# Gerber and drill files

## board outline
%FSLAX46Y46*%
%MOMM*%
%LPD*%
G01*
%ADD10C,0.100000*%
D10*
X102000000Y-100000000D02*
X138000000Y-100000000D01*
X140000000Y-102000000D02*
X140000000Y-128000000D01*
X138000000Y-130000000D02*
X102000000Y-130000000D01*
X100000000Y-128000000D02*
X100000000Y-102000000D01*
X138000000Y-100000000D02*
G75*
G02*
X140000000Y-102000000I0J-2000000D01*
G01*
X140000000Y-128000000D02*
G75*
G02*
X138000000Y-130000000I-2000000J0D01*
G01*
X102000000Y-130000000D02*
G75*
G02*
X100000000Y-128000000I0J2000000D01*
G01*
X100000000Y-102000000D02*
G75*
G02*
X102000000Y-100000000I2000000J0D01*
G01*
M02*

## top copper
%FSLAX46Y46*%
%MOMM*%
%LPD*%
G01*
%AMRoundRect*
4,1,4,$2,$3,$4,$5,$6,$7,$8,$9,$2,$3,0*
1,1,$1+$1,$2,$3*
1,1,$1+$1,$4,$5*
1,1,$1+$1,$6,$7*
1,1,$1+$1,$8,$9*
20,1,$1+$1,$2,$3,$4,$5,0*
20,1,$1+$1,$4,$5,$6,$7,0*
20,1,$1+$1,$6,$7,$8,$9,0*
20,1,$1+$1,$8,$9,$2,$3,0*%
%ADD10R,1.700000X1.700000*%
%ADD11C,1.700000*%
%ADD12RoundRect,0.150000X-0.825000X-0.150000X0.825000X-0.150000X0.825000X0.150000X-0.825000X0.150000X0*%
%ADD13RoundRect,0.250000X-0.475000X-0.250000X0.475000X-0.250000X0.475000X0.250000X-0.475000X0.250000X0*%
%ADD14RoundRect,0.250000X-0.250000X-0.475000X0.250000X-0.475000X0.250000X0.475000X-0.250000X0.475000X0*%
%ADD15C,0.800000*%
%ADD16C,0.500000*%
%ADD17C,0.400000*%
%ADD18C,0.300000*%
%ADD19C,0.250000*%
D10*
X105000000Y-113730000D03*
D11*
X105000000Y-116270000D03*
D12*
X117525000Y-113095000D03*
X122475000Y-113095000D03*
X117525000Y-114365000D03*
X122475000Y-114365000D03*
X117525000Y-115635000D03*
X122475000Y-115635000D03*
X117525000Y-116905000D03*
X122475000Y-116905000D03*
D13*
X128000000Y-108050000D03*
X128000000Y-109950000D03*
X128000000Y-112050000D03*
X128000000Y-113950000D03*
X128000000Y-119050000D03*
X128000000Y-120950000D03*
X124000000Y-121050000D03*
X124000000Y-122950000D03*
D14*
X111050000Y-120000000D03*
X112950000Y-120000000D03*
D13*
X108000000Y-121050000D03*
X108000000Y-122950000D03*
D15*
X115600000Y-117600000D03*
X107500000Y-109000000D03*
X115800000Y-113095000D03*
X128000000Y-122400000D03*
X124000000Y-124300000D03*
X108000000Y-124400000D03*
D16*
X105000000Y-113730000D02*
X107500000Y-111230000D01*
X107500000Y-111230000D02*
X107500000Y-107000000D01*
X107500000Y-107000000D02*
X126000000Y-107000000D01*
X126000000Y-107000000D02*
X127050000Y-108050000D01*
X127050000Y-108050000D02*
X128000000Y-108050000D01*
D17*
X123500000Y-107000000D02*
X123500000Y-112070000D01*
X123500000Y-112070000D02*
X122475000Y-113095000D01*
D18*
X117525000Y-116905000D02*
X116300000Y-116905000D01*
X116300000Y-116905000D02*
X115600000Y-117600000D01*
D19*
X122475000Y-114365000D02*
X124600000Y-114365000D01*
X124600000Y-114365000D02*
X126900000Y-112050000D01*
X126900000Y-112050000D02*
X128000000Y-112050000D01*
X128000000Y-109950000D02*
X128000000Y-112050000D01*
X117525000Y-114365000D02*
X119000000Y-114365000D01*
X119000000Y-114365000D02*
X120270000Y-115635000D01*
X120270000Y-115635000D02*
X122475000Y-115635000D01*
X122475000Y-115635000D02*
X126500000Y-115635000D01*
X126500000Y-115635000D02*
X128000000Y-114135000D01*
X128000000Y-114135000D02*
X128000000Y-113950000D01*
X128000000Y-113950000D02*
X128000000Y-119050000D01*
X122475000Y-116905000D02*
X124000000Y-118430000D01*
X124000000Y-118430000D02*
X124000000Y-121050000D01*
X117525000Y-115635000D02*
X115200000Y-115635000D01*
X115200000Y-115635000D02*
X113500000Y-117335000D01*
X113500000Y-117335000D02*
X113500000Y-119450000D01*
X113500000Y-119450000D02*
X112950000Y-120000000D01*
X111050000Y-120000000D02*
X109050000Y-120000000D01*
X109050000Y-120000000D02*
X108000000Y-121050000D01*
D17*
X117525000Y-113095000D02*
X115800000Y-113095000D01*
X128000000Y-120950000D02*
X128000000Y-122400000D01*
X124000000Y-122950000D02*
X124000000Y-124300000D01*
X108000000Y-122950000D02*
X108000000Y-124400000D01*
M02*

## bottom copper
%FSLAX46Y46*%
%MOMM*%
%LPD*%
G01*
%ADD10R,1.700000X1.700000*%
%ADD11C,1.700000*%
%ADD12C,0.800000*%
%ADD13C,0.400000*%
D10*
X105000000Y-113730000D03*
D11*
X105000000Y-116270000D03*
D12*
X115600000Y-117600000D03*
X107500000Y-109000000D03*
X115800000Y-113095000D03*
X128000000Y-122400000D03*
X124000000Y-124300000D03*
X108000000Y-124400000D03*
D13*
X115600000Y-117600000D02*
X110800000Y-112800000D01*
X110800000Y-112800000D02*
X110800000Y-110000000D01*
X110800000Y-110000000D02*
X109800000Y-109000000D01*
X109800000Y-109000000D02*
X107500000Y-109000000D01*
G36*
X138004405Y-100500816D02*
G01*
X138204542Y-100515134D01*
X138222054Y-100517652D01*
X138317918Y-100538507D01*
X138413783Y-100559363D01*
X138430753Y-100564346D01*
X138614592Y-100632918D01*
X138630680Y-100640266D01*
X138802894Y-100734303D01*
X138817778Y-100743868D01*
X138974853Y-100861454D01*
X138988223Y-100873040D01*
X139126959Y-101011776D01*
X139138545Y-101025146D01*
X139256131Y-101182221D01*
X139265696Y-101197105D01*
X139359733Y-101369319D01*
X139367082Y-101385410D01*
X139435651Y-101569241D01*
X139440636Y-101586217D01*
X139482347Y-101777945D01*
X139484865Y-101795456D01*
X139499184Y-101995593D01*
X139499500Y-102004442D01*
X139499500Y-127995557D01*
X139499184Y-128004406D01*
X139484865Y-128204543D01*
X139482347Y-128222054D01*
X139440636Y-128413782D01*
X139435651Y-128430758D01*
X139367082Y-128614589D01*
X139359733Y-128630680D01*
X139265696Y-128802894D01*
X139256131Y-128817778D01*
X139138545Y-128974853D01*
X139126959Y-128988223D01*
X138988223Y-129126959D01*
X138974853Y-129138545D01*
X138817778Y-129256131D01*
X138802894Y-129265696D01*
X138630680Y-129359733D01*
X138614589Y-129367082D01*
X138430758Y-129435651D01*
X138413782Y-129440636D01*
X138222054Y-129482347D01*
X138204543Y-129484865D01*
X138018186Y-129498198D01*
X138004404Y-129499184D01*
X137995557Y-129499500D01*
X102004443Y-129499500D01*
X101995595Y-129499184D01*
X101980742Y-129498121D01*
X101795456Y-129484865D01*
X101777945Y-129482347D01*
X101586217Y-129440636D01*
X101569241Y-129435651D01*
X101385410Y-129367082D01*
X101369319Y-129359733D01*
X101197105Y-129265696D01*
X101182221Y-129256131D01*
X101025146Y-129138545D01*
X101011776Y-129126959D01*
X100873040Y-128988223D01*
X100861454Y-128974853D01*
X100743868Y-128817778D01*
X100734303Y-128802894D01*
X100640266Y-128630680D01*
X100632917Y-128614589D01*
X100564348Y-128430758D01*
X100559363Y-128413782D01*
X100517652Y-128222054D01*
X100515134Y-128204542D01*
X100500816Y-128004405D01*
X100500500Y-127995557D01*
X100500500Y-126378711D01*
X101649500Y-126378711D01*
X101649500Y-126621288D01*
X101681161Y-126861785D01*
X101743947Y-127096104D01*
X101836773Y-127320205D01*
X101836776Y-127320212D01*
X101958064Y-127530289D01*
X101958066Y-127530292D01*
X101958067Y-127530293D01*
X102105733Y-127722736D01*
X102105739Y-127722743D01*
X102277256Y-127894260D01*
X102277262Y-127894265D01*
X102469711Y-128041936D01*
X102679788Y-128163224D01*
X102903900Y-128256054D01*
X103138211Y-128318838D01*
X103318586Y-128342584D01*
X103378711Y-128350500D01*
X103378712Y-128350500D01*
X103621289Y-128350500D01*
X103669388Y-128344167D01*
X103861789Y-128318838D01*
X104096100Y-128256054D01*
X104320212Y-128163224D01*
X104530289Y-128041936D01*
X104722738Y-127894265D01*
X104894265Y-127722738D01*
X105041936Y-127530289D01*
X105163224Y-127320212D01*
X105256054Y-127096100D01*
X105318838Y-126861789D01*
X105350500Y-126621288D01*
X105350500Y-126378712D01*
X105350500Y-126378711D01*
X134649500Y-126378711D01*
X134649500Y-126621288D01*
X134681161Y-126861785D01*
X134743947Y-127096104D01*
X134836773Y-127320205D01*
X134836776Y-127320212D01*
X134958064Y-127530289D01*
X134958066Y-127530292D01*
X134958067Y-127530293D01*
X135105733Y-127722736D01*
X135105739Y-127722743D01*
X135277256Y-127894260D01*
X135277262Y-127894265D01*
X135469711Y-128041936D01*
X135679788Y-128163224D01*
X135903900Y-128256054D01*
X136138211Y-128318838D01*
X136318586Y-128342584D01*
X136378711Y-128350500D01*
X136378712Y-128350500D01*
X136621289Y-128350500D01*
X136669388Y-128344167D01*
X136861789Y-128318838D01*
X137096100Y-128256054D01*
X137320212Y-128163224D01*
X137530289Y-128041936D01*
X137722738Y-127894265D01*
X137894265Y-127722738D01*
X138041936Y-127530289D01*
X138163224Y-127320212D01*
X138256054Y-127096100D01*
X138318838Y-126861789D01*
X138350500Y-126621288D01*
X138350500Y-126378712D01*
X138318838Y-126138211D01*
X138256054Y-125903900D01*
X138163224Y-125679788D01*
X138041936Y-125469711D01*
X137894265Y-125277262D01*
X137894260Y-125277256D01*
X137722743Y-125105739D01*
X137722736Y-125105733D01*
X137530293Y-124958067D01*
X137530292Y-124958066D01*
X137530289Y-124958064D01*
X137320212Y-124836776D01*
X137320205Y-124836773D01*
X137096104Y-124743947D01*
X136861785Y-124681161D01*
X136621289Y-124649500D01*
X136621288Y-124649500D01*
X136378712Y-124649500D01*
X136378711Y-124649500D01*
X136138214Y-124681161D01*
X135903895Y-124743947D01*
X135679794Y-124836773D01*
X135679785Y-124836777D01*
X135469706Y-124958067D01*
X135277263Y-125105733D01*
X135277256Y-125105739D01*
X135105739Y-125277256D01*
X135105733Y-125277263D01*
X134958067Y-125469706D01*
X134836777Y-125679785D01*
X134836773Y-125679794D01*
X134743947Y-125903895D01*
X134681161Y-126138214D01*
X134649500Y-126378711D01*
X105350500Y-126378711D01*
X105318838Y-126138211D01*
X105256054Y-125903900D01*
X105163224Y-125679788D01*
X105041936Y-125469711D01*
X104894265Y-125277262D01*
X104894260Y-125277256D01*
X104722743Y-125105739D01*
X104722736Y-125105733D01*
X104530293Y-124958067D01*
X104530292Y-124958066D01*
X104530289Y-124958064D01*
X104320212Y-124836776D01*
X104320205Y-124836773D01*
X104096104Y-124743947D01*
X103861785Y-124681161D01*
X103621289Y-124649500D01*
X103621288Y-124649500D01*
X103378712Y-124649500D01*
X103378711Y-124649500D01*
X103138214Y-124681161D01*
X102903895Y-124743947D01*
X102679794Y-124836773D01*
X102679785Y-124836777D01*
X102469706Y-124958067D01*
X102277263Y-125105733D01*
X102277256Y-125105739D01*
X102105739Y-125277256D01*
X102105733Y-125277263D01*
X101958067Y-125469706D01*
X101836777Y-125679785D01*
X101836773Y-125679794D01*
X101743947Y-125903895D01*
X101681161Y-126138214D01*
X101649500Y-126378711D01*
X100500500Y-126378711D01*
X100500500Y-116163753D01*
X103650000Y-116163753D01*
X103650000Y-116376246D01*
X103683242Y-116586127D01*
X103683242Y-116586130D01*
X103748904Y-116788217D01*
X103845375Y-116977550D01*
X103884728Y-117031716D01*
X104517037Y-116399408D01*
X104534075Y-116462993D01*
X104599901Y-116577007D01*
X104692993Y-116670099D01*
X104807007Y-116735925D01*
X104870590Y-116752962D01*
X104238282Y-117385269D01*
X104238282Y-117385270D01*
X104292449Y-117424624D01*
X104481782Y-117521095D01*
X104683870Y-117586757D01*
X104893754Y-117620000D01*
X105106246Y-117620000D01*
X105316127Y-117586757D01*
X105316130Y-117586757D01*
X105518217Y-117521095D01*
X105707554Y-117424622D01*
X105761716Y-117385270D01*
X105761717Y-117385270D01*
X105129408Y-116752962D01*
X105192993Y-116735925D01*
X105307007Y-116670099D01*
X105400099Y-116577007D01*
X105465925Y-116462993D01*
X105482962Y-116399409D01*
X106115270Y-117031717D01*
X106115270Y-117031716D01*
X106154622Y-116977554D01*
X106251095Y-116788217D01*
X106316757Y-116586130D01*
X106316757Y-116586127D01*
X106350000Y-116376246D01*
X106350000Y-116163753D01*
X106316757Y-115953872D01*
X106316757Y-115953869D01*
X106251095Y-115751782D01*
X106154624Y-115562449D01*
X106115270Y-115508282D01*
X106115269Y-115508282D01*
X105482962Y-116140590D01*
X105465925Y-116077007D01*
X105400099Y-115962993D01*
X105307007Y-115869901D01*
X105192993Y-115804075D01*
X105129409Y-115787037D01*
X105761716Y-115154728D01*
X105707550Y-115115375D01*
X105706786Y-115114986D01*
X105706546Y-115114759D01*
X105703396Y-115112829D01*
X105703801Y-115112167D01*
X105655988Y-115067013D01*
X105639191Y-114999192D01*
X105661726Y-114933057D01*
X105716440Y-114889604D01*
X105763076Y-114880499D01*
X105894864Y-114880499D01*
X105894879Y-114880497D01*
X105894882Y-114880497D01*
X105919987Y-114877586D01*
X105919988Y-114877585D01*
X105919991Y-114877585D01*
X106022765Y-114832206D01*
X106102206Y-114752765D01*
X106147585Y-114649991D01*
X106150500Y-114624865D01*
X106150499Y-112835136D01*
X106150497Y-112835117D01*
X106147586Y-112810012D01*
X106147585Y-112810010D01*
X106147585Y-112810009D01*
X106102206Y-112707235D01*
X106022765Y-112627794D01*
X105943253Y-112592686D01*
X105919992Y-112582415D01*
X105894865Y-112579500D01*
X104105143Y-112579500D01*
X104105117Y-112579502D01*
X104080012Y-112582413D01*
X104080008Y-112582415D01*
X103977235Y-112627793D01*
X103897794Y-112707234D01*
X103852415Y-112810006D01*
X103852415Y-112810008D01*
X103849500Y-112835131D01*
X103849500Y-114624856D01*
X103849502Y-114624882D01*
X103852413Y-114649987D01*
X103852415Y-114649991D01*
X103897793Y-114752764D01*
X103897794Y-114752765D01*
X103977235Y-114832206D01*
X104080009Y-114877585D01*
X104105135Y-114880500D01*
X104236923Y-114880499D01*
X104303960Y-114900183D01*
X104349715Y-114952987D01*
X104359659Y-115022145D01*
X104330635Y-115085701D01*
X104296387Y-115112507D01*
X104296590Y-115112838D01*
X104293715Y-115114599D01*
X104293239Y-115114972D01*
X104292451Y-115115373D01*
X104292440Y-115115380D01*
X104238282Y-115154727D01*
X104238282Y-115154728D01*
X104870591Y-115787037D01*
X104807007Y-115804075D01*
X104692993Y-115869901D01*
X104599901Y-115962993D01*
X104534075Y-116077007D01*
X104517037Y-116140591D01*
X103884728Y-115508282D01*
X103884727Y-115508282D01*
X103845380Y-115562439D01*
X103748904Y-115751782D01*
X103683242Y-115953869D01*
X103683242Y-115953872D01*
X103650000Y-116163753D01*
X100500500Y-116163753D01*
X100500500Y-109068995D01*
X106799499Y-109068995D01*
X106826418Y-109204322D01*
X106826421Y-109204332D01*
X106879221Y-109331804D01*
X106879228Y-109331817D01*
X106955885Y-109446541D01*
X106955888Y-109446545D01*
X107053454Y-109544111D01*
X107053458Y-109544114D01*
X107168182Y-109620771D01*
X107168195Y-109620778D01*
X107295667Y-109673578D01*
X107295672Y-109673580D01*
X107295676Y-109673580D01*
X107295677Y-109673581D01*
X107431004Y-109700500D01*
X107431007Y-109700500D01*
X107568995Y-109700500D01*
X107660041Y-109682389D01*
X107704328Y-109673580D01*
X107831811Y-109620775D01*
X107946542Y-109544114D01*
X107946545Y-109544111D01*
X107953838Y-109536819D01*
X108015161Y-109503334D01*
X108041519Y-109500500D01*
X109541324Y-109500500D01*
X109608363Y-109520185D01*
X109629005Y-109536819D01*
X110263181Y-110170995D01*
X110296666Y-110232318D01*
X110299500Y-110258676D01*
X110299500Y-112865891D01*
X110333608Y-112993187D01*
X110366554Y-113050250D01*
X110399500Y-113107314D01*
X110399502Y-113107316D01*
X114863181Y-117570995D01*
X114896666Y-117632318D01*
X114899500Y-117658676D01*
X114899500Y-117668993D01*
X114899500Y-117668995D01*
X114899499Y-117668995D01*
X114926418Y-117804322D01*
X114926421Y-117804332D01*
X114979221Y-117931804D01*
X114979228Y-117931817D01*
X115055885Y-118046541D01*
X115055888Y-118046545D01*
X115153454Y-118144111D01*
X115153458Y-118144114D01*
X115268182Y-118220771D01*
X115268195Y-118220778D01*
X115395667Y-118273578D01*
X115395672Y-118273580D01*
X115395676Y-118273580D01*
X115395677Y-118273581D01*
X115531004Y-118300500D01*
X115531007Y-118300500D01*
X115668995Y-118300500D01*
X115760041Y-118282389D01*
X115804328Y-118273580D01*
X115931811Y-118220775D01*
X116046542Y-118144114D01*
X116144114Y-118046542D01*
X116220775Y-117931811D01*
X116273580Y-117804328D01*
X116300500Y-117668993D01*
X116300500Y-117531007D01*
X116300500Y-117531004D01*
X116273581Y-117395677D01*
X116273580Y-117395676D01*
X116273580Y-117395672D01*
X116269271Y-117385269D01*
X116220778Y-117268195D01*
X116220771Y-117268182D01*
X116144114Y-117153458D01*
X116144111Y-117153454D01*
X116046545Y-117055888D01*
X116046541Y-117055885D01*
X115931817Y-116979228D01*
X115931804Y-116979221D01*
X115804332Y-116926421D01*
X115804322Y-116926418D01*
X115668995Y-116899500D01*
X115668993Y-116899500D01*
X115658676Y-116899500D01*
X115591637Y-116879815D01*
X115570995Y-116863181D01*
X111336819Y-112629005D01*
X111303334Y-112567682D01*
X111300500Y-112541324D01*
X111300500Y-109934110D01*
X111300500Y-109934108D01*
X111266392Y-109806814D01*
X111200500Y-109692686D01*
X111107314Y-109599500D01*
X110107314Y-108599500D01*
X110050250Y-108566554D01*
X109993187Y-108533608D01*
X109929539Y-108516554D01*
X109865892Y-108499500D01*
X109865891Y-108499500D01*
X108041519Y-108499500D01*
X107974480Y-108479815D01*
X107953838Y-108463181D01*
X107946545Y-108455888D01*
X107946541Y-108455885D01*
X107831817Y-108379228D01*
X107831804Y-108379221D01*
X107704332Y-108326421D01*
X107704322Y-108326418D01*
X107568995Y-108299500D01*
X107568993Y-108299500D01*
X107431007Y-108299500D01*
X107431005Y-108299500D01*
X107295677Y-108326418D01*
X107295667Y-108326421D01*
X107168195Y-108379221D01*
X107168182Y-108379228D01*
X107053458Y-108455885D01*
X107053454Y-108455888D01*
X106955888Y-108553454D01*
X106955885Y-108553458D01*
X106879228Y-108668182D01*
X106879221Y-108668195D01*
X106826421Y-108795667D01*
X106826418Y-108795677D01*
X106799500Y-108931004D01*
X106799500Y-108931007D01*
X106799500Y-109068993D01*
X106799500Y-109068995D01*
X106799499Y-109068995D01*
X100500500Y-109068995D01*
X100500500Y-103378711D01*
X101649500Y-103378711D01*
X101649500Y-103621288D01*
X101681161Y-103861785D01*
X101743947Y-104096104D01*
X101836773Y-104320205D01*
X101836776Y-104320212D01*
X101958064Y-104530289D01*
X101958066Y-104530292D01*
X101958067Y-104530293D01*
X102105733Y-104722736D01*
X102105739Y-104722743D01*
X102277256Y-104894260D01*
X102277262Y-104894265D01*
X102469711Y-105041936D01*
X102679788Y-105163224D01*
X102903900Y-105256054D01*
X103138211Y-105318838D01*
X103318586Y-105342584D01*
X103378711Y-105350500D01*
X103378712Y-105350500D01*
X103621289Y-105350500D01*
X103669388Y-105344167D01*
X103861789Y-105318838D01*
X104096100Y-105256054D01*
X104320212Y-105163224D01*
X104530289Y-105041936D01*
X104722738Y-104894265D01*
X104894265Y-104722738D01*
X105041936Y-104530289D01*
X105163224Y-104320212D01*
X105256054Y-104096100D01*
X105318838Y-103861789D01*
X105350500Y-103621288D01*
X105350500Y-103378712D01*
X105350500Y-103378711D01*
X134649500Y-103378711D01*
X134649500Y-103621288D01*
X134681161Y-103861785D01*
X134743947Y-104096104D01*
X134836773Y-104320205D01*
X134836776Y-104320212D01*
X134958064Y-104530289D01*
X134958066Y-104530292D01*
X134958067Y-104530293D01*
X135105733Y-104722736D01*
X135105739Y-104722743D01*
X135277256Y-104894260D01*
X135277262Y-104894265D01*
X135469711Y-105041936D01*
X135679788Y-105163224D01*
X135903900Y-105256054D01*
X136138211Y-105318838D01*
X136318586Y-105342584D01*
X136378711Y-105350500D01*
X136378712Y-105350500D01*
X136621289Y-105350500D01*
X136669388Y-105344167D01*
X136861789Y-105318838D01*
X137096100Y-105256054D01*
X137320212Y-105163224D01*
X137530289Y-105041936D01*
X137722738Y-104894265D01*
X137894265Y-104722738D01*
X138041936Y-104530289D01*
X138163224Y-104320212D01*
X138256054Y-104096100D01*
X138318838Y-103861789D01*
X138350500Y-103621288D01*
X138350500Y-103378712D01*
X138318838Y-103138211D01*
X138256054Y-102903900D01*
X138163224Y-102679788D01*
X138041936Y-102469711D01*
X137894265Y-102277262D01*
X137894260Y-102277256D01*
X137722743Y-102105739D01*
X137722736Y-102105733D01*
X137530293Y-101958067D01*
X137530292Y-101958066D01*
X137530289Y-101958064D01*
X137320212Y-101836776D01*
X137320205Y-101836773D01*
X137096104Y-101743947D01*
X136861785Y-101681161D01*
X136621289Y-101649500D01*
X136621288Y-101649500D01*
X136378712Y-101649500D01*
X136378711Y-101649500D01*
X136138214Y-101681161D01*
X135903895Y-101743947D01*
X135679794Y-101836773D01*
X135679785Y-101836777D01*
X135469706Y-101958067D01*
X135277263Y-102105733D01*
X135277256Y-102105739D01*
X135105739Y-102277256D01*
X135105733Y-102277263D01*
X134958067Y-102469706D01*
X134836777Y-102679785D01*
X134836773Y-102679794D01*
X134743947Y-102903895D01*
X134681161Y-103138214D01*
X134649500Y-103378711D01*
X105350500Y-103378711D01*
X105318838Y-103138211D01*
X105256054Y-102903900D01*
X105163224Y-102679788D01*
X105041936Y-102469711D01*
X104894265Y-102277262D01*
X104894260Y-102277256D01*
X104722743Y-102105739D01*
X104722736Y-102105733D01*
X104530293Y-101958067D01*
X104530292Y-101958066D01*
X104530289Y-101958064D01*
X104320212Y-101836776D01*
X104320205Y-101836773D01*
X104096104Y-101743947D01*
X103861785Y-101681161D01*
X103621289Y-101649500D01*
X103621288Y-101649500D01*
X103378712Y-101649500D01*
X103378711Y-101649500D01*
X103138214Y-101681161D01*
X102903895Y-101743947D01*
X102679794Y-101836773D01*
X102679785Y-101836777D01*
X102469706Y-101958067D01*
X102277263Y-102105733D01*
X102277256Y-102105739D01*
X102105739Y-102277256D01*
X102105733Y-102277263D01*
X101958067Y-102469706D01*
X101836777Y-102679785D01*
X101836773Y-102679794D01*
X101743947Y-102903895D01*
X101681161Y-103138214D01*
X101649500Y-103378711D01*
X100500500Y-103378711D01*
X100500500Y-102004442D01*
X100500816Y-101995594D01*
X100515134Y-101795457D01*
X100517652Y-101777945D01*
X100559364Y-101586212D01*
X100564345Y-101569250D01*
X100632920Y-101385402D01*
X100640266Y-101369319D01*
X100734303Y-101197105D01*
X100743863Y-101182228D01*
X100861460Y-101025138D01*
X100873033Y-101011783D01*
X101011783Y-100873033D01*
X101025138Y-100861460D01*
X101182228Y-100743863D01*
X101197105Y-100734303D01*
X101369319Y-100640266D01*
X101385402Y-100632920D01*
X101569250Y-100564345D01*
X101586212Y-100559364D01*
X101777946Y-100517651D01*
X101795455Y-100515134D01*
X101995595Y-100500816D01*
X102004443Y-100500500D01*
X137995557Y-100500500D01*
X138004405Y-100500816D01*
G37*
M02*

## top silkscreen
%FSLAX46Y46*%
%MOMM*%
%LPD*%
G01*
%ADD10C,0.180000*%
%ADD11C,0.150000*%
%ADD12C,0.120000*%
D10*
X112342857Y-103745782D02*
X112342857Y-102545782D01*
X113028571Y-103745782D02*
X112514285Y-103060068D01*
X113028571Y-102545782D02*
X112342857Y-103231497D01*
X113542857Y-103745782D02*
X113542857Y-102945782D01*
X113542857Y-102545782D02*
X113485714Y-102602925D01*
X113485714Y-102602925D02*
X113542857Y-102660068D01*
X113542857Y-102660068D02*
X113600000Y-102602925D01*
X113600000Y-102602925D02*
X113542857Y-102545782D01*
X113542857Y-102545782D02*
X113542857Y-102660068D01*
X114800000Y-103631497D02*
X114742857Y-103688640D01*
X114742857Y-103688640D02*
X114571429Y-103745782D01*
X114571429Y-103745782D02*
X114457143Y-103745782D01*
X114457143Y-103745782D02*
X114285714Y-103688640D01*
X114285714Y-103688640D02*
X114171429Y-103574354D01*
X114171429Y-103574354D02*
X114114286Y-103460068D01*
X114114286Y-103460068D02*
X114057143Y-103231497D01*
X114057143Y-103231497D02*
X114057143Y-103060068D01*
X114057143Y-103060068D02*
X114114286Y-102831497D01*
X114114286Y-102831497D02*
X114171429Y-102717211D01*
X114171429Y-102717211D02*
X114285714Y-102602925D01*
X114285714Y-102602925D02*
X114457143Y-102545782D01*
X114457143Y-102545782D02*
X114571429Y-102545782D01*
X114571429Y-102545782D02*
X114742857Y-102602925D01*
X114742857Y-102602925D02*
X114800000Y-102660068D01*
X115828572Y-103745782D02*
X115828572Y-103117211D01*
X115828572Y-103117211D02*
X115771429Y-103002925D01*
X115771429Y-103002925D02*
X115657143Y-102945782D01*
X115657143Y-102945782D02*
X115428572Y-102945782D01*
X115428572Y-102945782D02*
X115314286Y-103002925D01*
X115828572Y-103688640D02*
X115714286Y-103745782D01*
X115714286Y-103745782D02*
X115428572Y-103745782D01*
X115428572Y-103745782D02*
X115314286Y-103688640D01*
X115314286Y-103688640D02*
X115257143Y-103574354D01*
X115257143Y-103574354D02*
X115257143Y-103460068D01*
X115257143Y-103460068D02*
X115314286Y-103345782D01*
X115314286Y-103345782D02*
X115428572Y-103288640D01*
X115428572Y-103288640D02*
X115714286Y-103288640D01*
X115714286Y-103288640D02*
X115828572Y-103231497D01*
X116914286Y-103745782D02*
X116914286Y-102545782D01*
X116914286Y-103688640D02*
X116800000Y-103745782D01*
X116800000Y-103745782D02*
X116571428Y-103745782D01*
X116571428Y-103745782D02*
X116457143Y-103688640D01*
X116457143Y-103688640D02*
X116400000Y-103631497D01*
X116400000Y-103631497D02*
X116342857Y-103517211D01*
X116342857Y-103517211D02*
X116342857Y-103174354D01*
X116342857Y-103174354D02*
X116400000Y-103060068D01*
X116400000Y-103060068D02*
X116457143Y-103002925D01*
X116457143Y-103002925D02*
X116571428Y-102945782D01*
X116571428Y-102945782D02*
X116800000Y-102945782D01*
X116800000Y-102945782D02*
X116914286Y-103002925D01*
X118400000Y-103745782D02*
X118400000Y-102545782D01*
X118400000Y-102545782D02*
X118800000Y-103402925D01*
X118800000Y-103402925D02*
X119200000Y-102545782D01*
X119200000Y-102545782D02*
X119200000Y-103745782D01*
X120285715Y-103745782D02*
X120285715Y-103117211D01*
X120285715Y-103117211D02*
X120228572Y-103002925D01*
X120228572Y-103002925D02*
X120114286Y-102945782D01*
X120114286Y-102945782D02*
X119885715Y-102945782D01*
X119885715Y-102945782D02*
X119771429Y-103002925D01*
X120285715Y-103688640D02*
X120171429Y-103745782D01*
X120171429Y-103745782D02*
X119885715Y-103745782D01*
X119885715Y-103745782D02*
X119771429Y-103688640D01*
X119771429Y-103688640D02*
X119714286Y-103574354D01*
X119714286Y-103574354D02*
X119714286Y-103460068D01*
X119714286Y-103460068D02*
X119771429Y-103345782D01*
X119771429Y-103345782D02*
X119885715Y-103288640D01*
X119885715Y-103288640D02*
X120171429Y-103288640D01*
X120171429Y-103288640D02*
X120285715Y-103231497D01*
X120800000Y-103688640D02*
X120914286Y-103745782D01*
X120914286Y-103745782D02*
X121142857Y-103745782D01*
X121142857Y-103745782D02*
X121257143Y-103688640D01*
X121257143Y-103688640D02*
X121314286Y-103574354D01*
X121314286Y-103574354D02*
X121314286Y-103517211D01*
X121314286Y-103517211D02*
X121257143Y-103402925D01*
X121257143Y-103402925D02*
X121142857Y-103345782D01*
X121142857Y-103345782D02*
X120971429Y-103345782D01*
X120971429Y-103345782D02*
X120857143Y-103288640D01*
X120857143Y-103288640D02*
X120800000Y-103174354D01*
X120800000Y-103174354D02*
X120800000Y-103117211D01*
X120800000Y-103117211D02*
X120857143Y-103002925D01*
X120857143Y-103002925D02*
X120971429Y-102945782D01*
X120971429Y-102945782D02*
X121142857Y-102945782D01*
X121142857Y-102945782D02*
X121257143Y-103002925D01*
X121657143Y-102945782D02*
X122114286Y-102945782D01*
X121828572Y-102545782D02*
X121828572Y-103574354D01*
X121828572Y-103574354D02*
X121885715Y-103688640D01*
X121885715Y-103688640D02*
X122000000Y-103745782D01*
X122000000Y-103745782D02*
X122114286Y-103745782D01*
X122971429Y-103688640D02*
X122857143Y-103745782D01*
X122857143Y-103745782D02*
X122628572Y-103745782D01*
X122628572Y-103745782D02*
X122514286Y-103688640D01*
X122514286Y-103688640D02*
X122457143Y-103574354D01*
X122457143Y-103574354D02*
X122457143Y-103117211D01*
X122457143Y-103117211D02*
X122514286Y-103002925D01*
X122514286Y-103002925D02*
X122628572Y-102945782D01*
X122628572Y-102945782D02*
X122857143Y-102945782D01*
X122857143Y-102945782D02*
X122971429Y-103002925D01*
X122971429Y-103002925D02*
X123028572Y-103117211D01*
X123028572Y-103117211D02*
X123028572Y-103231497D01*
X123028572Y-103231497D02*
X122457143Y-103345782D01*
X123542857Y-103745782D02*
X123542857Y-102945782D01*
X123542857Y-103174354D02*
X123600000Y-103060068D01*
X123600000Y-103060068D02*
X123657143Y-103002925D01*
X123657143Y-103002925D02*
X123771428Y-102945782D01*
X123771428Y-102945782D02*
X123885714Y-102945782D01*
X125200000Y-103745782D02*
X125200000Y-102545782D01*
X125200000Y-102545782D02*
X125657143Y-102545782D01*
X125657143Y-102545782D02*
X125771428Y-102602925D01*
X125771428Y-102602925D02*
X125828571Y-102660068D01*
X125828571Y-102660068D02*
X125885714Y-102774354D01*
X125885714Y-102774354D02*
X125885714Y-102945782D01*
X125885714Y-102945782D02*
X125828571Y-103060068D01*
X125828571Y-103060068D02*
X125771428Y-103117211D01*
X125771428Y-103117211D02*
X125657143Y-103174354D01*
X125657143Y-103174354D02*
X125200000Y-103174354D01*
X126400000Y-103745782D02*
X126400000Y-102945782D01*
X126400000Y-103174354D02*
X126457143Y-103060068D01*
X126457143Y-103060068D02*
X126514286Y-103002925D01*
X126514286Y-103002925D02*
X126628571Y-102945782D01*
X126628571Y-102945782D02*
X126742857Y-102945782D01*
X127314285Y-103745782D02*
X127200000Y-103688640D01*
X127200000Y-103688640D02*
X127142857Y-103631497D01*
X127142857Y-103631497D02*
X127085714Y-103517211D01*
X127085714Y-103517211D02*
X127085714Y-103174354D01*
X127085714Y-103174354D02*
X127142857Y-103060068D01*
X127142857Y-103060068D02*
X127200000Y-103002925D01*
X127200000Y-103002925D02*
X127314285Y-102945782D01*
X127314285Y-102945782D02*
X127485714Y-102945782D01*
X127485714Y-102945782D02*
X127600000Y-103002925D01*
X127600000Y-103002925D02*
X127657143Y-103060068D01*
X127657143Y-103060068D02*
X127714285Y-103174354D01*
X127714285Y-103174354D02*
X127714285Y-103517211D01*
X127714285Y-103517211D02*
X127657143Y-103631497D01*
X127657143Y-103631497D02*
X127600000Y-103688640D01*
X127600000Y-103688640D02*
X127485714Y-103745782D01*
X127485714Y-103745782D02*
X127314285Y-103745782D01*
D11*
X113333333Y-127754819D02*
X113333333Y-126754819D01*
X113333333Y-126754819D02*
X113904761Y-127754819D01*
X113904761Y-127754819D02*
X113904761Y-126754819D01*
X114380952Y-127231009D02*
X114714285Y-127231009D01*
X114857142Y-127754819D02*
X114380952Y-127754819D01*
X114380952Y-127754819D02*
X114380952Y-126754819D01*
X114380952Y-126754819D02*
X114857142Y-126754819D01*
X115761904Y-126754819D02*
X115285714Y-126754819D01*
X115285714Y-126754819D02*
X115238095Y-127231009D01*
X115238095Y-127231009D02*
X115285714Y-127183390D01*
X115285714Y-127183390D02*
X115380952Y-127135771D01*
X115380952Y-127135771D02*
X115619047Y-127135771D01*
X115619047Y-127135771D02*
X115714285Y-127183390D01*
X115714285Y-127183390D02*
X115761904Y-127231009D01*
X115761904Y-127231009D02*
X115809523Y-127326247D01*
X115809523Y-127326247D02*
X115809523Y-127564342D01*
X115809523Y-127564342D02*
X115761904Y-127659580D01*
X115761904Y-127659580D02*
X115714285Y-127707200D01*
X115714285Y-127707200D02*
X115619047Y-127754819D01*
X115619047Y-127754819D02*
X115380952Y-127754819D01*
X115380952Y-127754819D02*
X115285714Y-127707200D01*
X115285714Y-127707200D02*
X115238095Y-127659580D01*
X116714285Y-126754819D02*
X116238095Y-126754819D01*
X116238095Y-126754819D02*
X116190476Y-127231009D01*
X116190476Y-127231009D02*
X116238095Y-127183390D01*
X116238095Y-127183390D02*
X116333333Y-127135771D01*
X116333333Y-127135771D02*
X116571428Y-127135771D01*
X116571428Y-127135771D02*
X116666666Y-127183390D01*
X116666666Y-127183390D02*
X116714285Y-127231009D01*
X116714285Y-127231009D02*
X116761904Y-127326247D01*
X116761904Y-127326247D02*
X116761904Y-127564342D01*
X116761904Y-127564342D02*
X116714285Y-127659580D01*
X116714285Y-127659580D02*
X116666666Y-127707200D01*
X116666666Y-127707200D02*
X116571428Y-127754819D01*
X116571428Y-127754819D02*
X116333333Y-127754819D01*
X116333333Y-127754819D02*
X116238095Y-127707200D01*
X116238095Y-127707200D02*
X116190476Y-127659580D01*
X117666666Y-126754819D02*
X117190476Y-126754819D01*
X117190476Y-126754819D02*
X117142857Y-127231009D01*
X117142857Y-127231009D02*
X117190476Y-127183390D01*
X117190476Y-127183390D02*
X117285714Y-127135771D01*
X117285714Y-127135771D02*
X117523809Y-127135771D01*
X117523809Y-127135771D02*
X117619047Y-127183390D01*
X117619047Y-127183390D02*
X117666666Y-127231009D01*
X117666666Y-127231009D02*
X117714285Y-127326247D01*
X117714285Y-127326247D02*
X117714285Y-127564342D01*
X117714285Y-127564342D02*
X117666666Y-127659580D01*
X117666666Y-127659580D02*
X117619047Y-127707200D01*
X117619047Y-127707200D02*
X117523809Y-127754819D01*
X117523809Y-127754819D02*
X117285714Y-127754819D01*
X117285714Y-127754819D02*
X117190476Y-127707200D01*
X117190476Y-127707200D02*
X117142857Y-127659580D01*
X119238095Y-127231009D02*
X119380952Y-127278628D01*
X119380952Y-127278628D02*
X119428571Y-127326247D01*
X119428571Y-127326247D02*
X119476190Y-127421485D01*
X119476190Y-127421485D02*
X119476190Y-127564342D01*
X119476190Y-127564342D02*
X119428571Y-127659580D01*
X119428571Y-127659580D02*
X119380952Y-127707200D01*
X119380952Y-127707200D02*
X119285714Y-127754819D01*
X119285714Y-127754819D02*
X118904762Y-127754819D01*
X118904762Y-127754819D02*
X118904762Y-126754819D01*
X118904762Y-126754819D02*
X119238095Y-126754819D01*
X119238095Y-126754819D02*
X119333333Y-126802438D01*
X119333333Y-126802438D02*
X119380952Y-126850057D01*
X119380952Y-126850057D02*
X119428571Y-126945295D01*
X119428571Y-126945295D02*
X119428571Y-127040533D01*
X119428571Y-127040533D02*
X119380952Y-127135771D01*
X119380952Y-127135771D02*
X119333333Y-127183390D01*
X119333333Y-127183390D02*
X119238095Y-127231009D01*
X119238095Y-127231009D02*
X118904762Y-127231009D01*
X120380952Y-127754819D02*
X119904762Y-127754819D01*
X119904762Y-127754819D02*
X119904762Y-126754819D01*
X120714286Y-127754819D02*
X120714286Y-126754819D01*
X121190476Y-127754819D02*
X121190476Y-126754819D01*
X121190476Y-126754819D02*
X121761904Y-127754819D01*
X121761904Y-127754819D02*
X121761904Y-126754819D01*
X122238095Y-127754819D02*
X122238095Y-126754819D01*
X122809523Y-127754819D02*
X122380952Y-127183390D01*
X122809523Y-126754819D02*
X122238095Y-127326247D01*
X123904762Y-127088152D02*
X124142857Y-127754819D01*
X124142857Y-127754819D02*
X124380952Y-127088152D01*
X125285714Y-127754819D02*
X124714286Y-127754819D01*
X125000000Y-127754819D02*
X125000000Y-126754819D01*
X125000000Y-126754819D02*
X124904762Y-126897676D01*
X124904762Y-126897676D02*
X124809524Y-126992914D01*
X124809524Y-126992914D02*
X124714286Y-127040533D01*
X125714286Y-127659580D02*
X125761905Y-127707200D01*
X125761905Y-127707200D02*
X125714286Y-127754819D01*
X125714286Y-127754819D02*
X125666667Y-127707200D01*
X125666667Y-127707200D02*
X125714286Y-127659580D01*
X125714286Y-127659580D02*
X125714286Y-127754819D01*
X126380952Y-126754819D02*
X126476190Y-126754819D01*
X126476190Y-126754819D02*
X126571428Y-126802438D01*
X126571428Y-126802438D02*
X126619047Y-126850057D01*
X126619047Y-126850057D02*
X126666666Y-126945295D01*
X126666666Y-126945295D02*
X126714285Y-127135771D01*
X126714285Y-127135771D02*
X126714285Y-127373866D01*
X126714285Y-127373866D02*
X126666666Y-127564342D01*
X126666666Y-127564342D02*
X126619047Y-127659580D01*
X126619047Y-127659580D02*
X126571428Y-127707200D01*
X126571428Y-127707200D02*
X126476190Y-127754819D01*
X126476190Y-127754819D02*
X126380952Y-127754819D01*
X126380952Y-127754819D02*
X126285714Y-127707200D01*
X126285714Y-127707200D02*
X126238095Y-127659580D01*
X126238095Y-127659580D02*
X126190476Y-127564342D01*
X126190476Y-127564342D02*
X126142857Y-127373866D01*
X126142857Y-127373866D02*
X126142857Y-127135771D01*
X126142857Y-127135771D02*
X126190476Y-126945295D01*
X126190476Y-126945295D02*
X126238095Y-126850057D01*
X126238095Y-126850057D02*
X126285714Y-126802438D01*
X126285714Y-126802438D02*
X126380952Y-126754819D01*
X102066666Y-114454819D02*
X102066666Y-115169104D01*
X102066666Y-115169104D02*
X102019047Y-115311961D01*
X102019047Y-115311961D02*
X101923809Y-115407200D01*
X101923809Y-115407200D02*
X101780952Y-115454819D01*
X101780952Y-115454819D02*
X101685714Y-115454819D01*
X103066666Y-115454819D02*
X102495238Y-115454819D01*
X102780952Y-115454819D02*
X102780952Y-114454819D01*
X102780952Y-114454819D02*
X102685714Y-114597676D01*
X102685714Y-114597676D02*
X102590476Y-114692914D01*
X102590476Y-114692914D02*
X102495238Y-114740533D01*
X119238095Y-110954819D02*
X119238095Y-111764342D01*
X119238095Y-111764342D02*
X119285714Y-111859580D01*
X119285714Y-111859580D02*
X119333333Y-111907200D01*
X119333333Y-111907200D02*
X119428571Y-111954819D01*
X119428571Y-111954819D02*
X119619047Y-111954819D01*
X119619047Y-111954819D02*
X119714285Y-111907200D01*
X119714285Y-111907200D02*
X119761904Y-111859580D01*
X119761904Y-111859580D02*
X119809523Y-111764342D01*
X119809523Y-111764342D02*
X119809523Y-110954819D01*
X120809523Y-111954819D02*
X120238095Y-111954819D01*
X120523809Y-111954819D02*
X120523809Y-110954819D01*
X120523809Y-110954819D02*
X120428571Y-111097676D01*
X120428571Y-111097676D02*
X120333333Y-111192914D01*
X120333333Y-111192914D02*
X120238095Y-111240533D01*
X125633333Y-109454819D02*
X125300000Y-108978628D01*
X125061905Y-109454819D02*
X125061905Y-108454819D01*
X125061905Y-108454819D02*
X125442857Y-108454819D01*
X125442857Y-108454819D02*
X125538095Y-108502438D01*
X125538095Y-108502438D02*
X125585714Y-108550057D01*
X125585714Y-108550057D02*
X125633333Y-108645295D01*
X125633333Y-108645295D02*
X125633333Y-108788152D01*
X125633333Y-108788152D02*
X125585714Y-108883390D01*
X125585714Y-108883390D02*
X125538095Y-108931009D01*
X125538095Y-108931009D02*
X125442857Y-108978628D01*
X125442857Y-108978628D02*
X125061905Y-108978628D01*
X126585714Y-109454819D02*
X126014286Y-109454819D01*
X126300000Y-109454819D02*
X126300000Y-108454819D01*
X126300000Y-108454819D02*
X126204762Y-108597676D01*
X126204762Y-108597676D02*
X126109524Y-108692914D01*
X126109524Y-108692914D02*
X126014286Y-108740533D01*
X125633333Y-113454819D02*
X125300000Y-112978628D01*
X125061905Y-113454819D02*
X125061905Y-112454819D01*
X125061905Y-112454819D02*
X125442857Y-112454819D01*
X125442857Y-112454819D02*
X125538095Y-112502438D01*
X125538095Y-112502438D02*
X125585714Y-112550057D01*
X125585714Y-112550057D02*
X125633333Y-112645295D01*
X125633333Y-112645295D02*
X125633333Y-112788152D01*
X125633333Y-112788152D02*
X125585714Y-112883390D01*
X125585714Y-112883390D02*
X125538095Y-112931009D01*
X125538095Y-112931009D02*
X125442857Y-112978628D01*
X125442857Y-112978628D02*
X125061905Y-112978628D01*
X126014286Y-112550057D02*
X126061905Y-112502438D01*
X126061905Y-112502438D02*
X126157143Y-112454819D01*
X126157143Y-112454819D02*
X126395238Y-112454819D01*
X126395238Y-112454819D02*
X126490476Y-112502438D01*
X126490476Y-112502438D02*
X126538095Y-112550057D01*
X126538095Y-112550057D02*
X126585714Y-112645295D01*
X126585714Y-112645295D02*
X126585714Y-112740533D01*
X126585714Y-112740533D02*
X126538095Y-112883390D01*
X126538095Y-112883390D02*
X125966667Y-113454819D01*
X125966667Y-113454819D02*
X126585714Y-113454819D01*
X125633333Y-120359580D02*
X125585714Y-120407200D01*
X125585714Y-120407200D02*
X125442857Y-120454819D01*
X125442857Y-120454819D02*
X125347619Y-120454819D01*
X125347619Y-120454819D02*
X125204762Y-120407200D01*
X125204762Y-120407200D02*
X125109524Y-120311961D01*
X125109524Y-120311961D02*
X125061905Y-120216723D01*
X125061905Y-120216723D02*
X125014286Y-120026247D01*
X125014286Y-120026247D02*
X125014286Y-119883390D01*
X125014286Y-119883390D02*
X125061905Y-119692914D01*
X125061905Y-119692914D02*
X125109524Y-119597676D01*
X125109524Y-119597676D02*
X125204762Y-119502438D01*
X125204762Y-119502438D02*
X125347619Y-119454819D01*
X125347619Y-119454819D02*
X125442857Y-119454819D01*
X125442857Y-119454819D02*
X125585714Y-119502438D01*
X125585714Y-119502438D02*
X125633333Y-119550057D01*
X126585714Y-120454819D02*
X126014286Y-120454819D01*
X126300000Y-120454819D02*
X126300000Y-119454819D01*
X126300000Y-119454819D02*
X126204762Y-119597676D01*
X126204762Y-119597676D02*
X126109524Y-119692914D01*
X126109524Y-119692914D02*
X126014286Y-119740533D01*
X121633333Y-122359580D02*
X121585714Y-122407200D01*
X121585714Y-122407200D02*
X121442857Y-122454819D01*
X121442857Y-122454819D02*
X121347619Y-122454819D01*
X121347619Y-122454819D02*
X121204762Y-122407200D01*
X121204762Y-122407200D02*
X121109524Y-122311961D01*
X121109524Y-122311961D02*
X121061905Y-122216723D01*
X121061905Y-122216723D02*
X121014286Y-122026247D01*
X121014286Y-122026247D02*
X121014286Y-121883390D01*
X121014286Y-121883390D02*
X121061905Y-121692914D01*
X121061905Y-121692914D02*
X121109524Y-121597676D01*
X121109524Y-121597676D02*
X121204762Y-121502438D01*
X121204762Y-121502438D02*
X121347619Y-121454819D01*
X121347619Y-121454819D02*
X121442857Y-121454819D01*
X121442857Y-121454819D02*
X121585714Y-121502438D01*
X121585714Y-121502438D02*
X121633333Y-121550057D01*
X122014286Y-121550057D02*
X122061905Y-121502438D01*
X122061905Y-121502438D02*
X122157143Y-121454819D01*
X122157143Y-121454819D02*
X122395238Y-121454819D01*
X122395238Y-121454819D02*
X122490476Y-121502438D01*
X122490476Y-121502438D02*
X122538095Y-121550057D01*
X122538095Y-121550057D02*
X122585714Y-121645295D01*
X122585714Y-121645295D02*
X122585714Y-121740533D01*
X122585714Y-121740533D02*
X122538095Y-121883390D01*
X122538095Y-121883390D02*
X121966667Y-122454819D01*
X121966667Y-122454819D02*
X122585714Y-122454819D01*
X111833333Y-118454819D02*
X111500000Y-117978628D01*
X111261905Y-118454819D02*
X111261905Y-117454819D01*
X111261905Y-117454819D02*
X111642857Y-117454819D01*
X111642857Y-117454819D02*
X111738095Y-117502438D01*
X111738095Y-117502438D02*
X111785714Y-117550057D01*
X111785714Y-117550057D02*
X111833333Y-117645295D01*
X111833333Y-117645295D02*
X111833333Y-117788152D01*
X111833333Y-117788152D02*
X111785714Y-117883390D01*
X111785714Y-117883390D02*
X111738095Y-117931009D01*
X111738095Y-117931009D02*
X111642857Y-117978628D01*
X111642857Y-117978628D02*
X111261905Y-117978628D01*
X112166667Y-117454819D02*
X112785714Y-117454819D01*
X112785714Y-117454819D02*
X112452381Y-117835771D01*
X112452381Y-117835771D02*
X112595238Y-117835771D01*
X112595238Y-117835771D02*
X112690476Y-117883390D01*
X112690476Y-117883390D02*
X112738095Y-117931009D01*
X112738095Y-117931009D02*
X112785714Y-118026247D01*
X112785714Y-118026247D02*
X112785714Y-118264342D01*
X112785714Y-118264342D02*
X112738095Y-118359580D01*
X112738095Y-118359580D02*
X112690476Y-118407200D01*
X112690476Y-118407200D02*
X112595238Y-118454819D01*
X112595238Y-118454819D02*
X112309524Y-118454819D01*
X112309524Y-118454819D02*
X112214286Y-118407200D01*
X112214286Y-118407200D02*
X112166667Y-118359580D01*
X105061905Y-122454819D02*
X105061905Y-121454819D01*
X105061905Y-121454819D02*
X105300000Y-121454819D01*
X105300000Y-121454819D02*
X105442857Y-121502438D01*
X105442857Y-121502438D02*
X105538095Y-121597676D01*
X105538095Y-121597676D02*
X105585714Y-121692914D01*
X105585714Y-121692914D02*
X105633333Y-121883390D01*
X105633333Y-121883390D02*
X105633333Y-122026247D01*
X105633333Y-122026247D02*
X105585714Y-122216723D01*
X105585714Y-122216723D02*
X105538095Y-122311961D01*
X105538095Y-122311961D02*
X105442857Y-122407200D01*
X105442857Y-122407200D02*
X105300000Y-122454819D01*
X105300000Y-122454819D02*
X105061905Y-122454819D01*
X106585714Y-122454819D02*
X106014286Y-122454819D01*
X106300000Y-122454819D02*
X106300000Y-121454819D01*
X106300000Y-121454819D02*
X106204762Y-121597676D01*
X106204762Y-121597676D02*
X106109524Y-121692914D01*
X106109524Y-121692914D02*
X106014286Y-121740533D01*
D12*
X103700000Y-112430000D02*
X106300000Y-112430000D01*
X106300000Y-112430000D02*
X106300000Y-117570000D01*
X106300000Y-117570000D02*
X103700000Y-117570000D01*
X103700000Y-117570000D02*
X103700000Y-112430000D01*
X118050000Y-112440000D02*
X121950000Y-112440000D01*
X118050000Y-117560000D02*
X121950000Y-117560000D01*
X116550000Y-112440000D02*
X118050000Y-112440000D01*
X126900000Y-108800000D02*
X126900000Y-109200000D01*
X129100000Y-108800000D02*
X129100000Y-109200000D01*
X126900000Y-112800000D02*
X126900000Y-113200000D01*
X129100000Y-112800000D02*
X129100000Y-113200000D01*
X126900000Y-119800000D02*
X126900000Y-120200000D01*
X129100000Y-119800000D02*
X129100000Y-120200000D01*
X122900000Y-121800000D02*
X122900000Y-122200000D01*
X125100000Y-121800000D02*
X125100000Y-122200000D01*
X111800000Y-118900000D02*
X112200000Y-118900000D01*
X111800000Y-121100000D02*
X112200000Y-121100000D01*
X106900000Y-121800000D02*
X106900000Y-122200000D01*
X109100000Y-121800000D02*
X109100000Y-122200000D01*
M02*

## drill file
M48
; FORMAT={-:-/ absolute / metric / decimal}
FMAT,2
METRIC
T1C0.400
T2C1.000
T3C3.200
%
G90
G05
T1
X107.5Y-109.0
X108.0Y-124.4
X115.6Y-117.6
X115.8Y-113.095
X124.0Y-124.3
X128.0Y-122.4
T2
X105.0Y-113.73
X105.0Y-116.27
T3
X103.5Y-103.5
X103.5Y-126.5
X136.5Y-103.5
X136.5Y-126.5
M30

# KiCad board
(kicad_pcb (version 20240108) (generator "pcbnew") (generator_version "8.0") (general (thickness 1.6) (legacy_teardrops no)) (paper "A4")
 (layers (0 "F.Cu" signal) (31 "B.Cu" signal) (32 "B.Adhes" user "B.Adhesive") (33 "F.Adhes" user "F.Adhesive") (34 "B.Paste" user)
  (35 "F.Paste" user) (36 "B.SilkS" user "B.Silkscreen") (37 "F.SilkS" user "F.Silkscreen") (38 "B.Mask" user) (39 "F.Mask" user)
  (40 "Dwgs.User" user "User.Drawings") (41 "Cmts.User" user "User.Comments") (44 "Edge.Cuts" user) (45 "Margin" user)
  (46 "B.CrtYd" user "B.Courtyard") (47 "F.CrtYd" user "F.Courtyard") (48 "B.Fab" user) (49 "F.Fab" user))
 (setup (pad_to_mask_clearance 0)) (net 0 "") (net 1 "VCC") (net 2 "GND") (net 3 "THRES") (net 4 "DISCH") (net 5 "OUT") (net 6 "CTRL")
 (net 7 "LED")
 (gr_line (start 102 100) (end 138 100) (stroke (width 0.1) (type default)) (layer "Edge.Cuts"))
 (gr_line (start 140 102) (end 140 128) (stroke (width 0.1) (type default)) (layer "Edge.Cuts"))
 (gr_line (start 138 130) (end 102 130) (stroke (width 0.1) (type default)) (layer "Edge.Cuts"))
 (gr_line (start 100 128) (end 100 102) (stroke (width 0.1) (type default)) (layer "Edge.Cuts"))
 (gr_arc (start 138 100) (mid 139.4142 100.5858) (end 140 102) (stroke (width 0.1) (type default)) (layer "Edge.Cuts"))
 (gr_arc (start 140 128) (mid 139.4142 129.4142) (end 138 130) (stroke (width 0.1) (type default)) (layer "Edge.Cuts"))
 (gr_arc (start 102 130) (mid 100.5858 129.4142) (end 100 128) (stroke (width 0.1) (type default)) (layer "Edge.Cuts"))
 (gr_arc (start 100 102) (mid 100.5858 100.5858) (end 102 100) (stroke (width 0.1) (type default)) (layer "Edge.Cuts"))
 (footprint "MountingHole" (layer "F.Cu") (at 103.5 103.5)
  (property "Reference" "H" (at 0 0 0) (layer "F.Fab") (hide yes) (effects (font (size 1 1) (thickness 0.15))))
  (pad "" np_thru_hole circle (at 0 0) (size 3.2 3.2) (drill 3.2) (layers "*.Cu" "*.Mask")))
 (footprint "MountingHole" (layer "F.Cu") (at 136.5 103.5)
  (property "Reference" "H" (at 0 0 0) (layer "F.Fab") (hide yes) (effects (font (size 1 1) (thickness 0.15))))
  (pad "" np_thru_hole circle (at 0 0) (size 3.2 3.2) (drill 3.2) (layers "*.Cu" "*.Mask")))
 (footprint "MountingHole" (layer "F.Cu") (at 103.5 126.5)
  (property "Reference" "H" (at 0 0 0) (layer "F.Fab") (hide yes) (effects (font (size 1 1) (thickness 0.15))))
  (pad "" np_thru_hole circle (at 0 0) (size 3.2 3.2) (drill 3.2) (layers "*.Cu" "*.Mask")))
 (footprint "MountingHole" (layer "F.Cu") (at 136.5 126.5)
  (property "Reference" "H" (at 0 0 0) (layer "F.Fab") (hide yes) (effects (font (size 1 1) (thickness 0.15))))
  (pad "" np_thru_hole circle (at 0 0) (size 3.2 3.2) (drill 3.2) (layers "*.Cu" "*.Mask")))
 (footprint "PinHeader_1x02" (layer "F.Cu") (at 105 113.73)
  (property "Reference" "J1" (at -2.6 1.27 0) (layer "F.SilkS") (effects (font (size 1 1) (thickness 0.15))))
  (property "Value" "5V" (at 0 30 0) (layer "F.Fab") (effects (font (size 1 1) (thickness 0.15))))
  (fp_line (start -1.3 -1.3) (end 1.3 -1.3) (stroke (width 0.12) (type solid)) (layer "F.SilkS"))
  (fp_line (start 1.3 -1.3) (end 1.3 3.84) (stroke (width 0.12) (type solid)) (layer "F.SilkS"))
  (fp_line (start 1.3 3.84) (end -1.3 3.84) (stroke (width 0.12) (type solid)) (layer "F.SilkS"))
  (fp_line (start -1.3 3.84) (end -1.3 -1.3) (stroke (width 0.12) (type solid)) (layer "F.SilkS"))
  (pad "1" thru_hole rect (at 0 0) (size 1.7 1.7) (drill 1) (layers "*.Cu" "*.Mask") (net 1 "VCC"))
  (pad "2" thru_hole circle (at 0 2.54) (size 1.7 1.7) (drill 1) (layers "*.Cu" "*.Mask") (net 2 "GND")))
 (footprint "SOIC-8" (layer "F.Cu") (at 120 115)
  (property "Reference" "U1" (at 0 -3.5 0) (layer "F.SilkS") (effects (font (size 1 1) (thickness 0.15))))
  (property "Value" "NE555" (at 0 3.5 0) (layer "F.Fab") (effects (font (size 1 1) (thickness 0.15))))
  (fp_line (start -1.95 -2.56) (end 1.95 -2.56) (stroke (width 0.12) (type solid)) (layer "F.SilkS"))
  (fp_line (start -1.95 2.56) (end 1.95 2.56) (stroke (width 0.12) (type solid)) (layer "F.SilkS"))
  (fp_line (start -3.45 -2.56) (end -1.95 -2.56) (stroke (width 0.12) (type solid)) (layer "F.SilkS"))
  (pad "1" smd roundrect (at -2.475 -1.905) (size 1.95 0.6) (layers "F.Cu" "F.Paste" "F.Mask") (roundrect_rratio 0.25) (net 2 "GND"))
  (pad "8" smd roundrect (at 2.475 -1.905) (size 1.95 0.6) (layers "F.Cu" "F.Paste" "F.Mask") (roundrect_rratio 0.25) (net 1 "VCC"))
  (pad "2" smd roundrect (at -2.475 -0.635) (size 1.95 0.6) (layers "F.Cu" "F.Paste" "F.Mask") (roundrect_rratio 0.25) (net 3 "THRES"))
  (pad "7" smd roundrect (at 2.475 -0.635) (size 1.95 0.6) (layers "F.Cu" "F.Paste" "F.Mask") (roundrect_rratio 0.25) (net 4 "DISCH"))
  (pad "3" smd roundrect (at -2.475 0.635) (size 1.95 0.6) (layers "F.Cu" "F.Paste" "F.Mask") (roundrect_rratio 0.25) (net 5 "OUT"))
  (pad "6" smd roundrect (at 2.475 0.635) (size 1.95 0.6) (layers "F.Cu" "F.Paste" "F.Mask") (roundrect_rratio 0.25) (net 3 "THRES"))
  (pad "4" smd roundrect (at -2.475 1.905) (size 1.95 0.6) (layers "F.Cu" "F.Paste" "F.Mask") (roundrect_rratio 0.25) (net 1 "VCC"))
  (pad "5" smd roundrect (at 2.475 1.905) (size 1.95 0.6) (layers "F.Cu" "F.Paste" "F.Mask") (roundrect_rratio 0.25) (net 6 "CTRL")))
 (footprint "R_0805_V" (layer "F.Cu") (at 128 109)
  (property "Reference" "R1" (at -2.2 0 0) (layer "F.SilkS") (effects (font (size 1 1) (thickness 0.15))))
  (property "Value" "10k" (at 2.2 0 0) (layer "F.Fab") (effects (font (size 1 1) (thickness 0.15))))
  (fp_line (start -1.1 -0.2) (end -1.1 0.2) (stroke (width 0.12) (type solid)) (layer "F.SilkS"))
  (fp_line (start 1.1 -0.2) (end 1.1 0.2) (stroke (width 0.12) (type solid)) (layer "F.SilkS"))
  (pad "1" smd roundrect (at 0 -0.95) (size 1.45 1) (layers "F.Cu" "F.Paste" "F.Mask") (roundrect_rratio 0.25) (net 1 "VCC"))
  (pad "2" smd roundrect (at 0 0.95) (size 1.45 1) (layers "F.Cu" "F.Paste" "F.Mask") (roundrect_rratio 0.25) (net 4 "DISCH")))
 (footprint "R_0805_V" (layer "F.Cu") (at 128 113)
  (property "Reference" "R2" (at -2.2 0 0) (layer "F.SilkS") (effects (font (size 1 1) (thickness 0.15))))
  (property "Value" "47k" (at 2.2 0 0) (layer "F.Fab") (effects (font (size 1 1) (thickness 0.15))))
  (fp_line (start -1.1 -0.2) (end -1.1 0.2) (stroke (width 0.12) (type solid)) (layer "F.SilkS"))
  (fp_line (start 1.1 -0.2) (end 1.1 0.2) (stroke (width 0.12) (type solid)) (layer "F.SilkS"))
  (pad "1" smd roundrect (at 0 -0.95) (size 1.45 1) (layers "F.Cu" "F.Paste" "F.Mask") (roundrect_rratio 0.25) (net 4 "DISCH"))
  (pad "2" smd roundrect (at 0 0.95) (size 1.45 1) (layers "F.Cu" "F.Paste" "F.Mask") (roundrect_rratio 0.25) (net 3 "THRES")))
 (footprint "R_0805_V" (layer "F.Cu") (at 128 120)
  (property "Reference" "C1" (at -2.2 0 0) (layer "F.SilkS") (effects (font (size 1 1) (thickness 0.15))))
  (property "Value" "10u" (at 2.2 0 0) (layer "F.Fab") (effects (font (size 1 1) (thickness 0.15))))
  (fp_line (start -1.1 -0.2) (end -1.1 0.2) (stroke (width 0.12) (type solid)) (layer "F.SilkS"))
  (fp_line (start 1.1 -0.2) (end 1.1 0.2) (stroke (width 0.12) (type solid)) (layer "F.SilkS"))
  (pad "1" smd roundrect (at 0 -0.95) (size 1.45 1) (layers "F.Cu" "F.Paste" "F.Mask") (roundrect_rratio 0.25) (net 3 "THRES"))
  (pad "2" smd roundrect (at 0 0.95) (size 1.45 1) (layers "F.Cu" "F.Paste" "F.Mask") (roundrect_rratio 0.25) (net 2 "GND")))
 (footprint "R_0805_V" (layer "F.Cu") (at 124 122)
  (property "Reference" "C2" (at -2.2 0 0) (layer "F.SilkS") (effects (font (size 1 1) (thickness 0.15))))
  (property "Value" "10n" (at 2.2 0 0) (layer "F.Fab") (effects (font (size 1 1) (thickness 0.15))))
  (fp_line (start -1.1 -0.2) (end -1.1 0.2) (stroke (width 0.12) (type solid)) (layer "F.SilkS"))
  (fp_line (start 1.1 -0.2) (end 1.1 0.2) (stroke (width 0.12) (type solid)) (layer "F.SilkS"))
  (pad "1" smd roundrect (at 0 -0.95) (size 1.45 1) (layers "F.Cu" "F.Paste" "F.Mask") (roundrect_rratio 0.25) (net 6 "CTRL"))
  (pad "2" smd roundrect (at 0 0.95) (size 1.45 1) (layers "F.Cu" "F.Paste" "F.Mask") (roundrect_rratio 0.25) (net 2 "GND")))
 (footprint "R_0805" (layer "F.Cu") (at 112 120)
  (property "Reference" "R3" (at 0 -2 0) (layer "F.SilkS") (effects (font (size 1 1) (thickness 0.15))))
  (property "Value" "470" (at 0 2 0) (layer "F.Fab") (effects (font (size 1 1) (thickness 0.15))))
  (fp_line (start -0.2 -1.1) (end 0.2 -1.1) (stroke (width 0.12) (type solid)) (layer "F.SilkS"))
  (fp_line (start -0.2 1.1) (end 0.2 1.1) (stroke (width 0.12) (type solid)) (layer "F.SilkS"))
  (pad "1" smd roundrect (at -0.95 0) (size 1 1.45) (layers "F.Cu" "F.Paste" "F.Mask") (roundrect_rratio 0.25) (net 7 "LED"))
  (pad "2" smd roundrect (at 0.95 0) (size 1 1.45) (layers "F.Cu" "F.Paste" "F.Mask") (roundrect_rratio 0.25) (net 5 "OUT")))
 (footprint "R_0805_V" (layer "F.Cu") (at 108 122)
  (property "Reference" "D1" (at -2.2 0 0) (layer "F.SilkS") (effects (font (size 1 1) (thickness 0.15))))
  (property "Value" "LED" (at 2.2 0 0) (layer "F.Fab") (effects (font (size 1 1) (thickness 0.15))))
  (fp_line (start -1.1 -0.2) (end -1.1 0.2) (stroke (width 0.12) (type solid)) (layer "F.SilkS"))
  (fp_line (start 1.1 -0.2) (end 1.1 0.2) (stroke (width 0.12) (type solid)) (layer "F.SilkS"))
  (pad "1" smd roundrect (at 0 -0.95) (size 1.45 1) (layers "F.Cu" "F.Paste" "F.Mask") (roundrect_rratio 0.25) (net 7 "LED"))
  (pad "2" smd roundrect (at 0 0.95) (size 1.45 1) (layers "F.Cu" "F.Paste" "F.Mask") (roundrect_rratio 0.25) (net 2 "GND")))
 (segment (start 105 113.73) (end 107.5 111.23) (width 0.5) (layer "F.Cu") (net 1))
 (segment (start 107.5 111.23) (end 107.5 107) (width 0.5) (layer "F.Cu") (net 1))
 (segment (start 107.5 107) (end 126 107) (width 0.5) (layer "F.Cu") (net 1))
 (segment (start 126 107) (end 127.05 108.05) (width 0.5) (layer "F.Cu") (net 1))
 (segment (start 127.05 108.05) (end 128 108.05) (width 0.5) (layer "F.Cu") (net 1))
 (segment (start 123.5 107) (end 123.5 112.07) (width 0.4) (layer "F.Cu") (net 1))
 (segment (start 123.5 112.07) (end 122.475 113.095) (width 0.4) (layer "F.Cu") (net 1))
 (segment (start 117.525 116.905) (end 116.3 116.905) (width 0.3) (layer "F.Cu") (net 1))
 (segment (start 116.3 116.905) (end 115.6 117.6) (width 0.3) (layer "F.Cu") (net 1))
 (via (at 115.6 117.6) (size 0.8) (drill 0.4) (layers "F.Cu" "B.Cu") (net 1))
 (via (at 107.5 109) (size 0.8) (drill 0.4) (layers "F.Cu" "B.Cu") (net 1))
 (segment (start 115.6 117.6) (end 110.8 112.8) (width 0.4) (layer "B.Cu") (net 1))
 (segment (start 110.8 112.8) (end 110.8 110) (width 0.4) (layer "B.Cu") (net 1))
 (segment (start 110.8 110) (end 109.8 109) (width 0.4) (layer "B.Cu") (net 1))
 (segment (start 109.8 109) (end 107.5 109) (width 0.4) (layer "B.Cu") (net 1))
 (segment (start 122.475 114.365) (end 124.6 114.365) (width 0.25) (layer "F.Cu") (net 4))
 (segment (start 124.6 114.365) (end 126.9 112.05) (width 0.25) (layer "F.Cu") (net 4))
 (segment (start 126.9 112.05) (end 128 112.05) (width 0.25) (layer "F.Cu") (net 4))
 (segment (start 128 109.95) (end 128 112.05) (width 0.25) (layer "F.Cu") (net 4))
 (segment (start 117.525 114.365) (end 119 114.365) (width 0.25) (layer "F.Cu") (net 3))
 (segment (start 119 114.365) (end 120.27 115.635) (width 0.25) (layer "F.Cu") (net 3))
 (segment (start 120.27 115.635) (end 122.475 115.635) (width 0.25) (layer "F.Cu") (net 3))
 (segment (start 122.475 115.635) (end 126.5 115.635) (width 0.25) (layer "F.Cu") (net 3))
 (segment (start 126.5 115.635) (end 128 114.135) (width 0.25) (layer "F.Cu") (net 3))
 (segment (start 128 114.135) (end 128 113.95) (width 0.25) (layer "F.Cu") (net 3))
 (segment (start 128 113.95) (end 128 119.05) (width 0.25) (layer "F.Cu") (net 3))
 (segment (start 122.475 116.905) (end 124 118.43) (width 0.25) (layer "F.Cu") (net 6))
 (segment (start 124 118.43) (end 124 121.05) (width 0.25) (layer "F.Cu") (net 6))
 (segment (start 117.525 115.635) (end 115.2 115.635) (width 0.25) (layer "F.Cu") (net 5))
 (segment (start 115.2 115.635) (end 113.5 117.335) (width 0.25) (layer "F.Cu") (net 5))
 (segment (start 113.5 117.335) (end 113.5 119.45) (width 0.25) (layer "F.Cu") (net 5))
 (segment (start 113.5 119.45) (end 112.95 120) (width 0.25) (layer "F.Cu") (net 5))
 (segment (start 111.05 120) (end 109.05 120) (width 0.25) (layer "F.Cu") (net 7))
 (segment (start 109.05 120) (end 108 121.05) (width 0.25) (layer "F.Cu") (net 7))
 (segment (start 117.525 113.095) (end 115.8 113.095) (width 0.4) (layer "F.Cu") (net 2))
 (via (at 115.8 113.095) (size 0.8) (drill 0.4) (layers "F.Cu" "B.Cu") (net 2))
 (segment (start 128 120.95) (end 128 122.4) (width 0.4) (layer "F.Cu") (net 2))
 (via (at 128 122.4) (size 0.8) (drill 0.4) (layers "F.Cu" "B.Cu") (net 2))
 (segment (start 124 122.95) (end 124 124.3) (width 0.4) (layer "F.Cu") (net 2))
 (via (at 124 124.3) (size 0.8) (drill 0.4) (layers "F.Cu" "B.Cu") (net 2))
 (segment (start 108 122.95) (end 108 124.4) (width 0.4) (layer "F.Cu") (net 2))
 (via (at 108 124.4) (size 0.8) (drill 0.4) (layers "F.Cu" "B.Cu") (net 2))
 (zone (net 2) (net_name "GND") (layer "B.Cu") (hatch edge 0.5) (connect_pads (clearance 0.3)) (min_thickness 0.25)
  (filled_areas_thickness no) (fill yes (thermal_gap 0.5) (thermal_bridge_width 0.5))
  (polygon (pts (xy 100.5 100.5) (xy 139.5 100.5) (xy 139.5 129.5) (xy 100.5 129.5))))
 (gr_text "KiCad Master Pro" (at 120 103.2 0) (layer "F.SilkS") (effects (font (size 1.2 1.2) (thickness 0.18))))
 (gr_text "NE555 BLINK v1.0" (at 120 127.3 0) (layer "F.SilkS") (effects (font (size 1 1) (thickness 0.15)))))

